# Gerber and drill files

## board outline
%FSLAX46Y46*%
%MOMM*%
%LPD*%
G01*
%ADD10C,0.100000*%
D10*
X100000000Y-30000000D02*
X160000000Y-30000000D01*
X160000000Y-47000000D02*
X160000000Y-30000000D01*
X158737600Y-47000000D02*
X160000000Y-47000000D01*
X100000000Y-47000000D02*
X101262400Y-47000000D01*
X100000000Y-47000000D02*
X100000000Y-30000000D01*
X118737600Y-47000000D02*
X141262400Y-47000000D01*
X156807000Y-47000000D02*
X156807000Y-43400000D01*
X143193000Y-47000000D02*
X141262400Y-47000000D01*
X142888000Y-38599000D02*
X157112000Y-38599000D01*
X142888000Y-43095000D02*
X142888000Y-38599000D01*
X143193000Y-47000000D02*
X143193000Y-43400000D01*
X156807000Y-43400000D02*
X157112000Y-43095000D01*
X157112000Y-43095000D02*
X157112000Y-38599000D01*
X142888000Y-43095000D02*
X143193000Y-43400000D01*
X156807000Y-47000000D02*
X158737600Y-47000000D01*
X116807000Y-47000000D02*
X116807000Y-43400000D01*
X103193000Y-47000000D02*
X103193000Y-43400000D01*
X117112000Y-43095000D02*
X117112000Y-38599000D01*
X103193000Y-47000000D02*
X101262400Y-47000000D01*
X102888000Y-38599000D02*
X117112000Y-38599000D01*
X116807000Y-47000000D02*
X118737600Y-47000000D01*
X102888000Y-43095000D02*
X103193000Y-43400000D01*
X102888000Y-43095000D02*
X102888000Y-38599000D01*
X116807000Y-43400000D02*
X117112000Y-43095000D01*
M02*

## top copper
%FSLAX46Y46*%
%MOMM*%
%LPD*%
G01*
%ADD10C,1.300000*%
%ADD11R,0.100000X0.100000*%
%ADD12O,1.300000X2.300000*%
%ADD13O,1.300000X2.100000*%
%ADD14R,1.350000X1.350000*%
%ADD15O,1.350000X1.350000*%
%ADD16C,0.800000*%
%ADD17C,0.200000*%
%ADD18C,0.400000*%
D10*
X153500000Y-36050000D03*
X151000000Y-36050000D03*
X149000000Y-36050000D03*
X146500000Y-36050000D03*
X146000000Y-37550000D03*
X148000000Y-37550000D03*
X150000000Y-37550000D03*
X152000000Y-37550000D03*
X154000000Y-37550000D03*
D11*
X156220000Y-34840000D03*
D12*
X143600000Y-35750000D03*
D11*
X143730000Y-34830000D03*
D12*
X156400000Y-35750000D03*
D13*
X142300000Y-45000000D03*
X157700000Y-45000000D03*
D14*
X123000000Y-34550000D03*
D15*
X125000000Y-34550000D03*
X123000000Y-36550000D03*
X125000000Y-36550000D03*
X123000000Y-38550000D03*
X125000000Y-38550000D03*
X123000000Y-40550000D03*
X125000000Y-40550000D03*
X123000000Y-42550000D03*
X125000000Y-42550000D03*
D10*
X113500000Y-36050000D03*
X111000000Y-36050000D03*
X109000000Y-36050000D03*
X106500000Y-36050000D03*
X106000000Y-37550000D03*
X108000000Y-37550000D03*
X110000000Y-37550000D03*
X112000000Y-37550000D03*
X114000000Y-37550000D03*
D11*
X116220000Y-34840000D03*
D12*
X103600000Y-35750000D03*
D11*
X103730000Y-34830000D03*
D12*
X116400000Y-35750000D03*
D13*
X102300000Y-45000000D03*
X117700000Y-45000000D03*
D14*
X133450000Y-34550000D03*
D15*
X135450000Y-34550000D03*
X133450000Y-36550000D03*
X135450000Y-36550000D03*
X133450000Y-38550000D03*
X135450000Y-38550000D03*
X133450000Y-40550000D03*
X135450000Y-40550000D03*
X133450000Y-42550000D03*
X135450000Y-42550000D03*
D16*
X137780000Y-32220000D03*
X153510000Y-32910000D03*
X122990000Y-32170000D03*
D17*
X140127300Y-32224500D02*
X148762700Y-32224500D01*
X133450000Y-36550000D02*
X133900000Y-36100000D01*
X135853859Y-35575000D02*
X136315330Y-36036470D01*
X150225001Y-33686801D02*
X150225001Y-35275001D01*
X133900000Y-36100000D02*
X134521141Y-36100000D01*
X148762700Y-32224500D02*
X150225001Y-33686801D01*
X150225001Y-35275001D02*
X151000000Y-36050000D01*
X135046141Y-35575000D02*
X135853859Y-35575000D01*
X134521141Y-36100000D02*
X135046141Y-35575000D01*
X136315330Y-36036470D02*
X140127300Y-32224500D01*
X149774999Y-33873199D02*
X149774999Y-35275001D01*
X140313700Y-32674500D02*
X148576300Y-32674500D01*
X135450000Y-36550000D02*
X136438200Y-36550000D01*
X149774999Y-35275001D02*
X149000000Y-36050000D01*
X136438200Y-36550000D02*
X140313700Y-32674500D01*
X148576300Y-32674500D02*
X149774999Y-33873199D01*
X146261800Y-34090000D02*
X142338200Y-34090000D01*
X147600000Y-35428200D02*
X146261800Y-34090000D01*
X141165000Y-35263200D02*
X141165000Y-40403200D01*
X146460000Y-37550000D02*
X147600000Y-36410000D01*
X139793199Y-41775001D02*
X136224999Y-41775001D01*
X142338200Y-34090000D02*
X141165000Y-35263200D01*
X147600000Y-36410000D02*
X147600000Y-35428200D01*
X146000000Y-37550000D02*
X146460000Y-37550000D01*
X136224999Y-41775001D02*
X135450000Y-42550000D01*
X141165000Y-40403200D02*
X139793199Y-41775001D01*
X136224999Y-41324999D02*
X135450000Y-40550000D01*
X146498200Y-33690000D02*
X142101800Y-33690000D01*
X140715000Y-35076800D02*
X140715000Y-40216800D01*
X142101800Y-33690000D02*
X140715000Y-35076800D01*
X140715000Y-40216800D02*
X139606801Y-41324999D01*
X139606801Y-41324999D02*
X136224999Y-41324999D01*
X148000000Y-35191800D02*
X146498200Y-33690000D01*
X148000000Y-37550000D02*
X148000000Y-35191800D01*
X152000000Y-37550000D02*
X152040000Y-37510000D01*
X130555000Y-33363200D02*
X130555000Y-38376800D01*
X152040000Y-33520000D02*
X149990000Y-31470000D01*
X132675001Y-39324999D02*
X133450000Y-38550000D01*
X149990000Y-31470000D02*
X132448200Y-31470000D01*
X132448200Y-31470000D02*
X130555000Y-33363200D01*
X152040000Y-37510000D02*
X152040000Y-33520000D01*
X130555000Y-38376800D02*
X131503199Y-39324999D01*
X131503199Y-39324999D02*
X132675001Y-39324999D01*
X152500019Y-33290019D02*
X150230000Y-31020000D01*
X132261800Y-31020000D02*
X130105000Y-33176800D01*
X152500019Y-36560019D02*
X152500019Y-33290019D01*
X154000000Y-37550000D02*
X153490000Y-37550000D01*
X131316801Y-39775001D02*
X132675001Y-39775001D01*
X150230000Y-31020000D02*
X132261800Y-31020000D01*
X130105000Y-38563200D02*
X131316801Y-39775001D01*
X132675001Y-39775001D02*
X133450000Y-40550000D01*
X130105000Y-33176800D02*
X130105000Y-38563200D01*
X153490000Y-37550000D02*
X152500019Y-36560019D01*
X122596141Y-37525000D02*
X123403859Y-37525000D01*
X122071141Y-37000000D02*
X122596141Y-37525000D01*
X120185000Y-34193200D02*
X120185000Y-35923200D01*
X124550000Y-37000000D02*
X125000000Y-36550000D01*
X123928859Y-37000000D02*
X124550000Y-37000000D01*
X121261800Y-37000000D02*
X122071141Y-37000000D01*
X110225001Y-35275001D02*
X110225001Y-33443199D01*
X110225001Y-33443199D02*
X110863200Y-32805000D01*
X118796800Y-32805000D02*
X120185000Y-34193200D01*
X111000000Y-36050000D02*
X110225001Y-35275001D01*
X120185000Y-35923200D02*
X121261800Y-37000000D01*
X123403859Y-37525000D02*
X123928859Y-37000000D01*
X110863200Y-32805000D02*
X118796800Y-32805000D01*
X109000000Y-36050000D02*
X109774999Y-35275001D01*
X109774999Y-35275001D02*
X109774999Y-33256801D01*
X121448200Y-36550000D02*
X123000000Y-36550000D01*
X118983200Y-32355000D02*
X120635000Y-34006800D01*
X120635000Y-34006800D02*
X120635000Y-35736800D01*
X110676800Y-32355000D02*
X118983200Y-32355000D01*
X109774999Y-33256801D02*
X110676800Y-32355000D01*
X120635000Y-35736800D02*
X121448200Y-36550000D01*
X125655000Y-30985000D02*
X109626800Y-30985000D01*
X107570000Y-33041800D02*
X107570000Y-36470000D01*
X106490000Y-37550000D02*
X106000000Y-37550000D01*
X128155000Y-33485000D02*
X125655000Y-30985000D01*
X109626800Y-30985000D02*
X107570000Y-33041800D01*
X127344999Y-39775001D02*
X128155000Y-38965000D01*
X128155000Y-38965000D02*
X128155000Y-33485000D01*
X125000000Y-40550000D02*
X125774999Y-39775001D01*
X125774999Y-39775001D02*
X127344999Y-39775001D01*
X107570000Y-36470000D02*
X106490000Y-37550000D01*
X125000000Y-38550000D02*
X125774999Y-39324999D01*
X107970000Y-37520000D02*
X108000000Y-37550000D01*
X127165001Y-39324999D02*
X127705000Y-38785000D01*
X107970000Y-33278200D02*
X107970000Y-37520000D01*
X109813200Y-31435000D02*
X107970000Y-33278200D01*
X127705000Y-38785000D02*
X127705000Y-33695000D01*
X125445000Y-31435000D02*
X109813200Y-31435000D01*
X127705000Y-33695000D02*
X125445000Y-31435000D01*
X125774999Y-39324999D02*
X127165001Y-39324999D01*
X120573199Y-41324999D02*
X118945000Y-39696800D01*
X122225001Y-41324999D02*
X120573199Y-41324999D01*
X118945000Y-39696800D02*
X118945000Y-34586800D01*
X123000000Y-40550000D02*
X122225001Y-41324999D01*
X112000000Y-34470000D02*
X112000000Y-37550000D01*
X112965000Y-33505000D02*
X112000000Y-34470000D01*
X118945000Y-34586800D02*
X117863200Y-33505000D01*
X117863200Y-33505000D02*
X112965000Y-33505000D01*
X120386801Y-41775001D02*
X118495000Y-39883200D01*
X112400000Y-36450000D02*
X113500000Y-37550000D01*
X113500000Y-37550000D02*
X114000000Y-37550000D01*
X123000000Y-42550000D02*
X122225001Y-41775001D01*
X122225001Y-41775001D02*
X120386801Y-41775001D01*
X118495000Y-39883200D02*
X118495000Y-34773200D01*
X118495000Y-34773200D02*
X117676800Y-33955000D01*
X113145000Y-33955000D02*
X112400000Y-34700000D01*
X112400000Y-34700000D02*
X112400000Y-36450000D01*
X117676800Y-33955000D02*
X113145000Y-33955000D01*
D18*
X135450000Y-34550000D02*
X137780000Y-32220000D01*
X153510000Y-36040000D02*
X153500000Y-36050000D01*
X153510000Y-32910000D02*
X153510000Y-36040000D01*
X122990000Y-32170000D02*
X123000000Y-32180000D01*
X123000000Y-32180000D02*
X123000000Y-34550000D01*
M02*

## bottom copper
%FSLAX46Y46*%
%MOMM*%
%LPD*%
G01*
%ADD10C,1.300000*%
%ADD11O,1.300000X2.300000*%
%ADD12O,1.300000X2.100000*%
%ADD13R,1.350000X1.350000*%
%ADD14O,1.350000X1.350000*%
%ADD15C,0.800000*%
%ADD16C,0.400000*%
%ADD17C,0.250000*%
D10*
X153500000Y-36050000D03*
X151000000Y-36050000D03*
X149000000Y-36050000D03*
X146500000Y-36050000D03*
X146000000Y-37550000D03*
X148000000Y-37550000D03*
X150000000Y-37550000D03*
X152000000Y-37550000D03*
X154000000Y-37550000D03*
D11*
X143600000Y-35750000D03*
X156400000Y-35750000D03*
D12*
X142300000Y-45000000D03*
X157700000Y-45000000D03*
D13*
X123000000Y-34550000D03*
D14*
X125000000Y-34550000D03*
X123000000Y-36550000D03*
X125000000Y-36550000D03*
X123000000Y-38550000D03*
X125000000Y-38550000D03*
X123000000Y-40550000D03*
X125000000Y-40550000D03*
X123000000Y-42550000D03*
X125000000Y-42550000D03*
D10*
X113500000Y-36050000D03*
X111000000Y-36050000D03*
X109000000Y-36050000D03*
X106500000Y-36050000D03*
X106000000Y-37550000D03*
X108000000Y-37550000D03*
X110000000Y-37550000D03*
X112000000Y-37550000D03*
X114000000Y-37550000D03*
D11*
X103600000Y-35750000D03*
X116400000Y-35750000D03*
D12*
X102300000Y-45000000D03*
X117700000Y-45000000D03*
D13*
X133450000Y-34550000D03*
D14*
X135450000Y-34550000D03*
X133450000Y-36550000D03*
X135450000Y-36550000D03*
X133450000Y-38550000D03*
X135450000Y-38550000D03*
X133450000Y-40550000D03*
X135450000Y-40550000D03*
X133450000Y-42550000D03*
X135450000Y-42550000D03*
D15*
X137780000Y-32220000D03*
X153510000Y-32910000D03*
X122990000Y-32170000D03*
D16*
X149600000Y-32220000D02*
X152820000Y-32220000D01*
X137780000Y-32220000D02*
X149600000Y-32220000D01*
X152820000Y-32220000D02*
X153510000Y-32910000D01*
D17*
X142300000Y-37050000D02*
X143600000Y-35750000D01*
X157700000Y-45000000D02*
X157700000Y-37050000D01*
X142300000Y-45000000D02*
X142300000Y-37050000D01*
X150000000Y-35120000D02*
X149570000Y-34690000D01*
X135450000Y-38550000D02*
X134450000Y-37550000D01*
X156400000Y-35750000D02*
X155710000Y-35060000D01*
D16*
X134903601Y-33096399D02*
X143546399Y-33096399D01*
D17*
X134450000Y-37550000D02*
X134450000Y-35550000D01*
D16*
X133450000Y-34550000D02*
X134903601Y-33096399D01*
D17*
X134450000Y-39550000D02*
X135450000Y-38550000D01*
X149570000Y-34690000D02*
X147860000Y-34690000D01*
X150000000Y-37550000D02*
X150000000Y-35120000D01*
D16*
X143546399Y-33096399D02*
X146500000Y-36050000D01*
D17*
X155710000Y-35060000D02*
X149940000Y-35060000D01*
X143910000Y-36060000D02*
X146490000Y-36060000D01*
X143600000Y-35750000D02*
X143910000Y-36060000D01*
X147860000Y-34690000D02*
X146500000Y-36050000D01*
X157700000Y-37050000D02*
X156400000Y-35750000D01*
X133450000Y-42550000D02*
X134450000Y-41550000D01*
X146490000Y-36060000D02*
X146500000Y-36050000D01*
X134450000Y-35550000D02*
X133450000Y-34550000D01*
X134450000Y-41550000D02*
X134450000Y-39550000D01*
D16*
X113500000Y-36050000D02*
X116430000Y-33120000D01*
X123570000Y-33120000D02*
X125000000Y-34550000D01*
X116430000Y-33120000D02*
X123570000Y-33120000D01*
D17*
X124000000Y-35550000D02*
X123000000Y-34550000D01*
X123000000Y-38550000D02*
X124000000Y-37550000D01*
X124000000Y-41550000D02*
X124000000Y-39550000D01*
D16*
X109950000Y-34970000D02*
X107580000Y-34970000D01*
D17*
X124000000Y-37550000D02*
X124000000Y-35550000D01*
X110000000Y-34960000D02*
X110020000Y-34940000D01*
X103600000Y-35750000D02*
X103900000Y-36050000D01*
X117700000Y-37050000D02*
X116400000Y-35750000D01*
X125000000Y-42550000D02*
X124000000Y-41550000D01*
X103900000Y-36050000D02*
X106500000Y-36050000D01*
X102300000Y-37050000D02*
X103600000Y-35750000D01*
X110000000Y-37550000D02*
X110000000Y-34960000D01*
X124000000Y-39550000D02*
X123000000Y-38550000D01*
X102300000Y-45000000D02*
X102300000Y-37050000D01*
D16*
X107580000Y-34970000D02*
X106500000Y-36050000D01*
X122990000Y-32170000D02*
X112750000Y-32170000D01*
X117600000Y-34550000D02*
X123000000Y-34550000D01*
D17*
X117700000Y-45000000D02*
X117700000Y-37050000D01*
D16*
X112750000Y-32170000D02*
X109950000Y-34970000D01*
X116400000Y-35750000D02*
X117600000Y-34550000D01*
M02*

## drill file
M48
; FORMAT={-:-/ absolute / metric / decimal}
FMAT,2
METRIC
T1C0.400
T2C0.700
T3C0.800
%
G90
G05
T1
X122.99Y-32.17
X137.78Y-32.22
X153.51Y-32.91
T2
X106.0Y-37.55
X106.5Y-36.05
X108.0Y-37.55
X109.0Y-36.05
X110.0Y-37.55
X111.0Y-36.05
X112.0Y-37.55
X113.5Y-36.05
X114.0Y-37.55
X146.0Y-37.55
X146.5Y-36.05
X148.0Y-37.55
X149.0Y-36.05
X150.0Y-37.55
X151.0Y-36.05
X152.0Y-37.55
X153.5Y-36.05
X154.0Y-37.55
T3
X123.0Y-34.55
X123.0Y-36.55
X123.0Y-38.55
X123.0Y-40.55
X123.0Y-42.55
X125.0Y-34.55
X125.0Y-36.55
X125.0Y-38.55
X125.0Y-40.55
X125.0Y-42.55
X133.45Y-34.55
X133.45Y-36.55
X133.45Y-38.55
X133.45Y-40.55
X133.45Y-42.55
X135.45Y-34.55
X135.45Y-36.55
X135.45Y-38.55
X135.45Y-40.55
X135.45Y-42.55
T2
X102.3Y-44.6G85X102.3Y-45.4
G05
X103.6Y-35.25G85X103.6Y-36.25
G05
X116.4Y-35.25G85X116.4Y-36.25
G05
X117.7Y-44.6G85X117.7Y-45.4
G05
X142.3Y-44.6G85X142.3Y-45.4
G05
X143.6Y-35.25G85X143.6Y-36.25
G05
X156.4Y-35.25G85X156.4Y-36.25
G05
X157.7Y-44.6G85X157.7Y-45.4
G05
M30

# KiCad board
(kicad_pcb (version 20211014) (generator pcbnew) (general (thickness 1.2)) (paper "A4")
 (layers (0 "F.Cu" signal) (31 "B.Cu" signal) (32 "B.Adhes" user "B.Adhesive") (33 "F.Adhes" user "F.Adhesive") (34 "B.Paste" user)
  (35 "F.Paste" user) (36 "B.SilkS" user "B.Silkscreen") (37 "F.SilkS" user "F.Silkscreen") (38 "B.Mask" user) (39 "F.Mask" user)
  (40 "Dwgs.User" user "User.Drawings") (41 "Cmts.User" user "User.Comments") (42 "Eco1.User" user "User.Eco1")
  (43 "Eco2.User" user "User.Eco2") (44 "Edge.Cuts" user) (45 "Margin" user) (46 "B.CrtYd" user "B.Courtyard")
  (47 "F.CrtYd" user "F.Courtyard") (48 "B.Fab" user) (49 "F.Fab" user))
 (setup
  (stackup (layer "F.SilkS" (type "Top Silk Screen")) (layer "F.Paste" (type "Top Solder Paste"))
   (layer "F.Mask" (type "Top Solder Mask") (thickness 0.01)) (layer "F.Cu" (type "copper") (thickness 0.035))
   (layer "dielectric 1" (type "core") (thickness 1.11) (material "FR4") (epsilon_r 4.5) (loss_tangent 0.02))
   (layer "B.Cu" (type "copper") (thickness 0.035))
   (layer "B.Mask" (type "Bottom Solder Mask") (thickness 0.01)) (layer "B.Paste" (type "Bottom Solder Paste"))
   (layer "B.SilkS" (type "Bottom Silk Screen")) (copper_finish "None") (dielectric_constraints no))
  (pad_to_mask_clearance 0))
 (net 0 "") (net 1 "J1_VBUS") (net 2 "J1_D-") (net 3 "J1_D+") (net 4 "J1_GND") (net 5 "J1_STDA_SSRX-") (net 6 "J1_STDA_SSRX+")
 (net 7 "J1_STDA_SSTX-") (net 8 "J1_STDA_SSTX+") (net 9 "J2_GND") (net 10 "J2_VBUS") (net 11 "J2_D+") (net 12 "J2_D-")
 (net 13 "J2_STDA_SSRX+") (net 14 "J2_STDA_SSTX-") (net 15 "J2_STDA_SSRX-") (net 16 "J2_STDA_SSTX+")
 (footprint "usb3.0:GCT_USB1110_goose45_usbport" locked (layer "F.Cu") (at 150 45)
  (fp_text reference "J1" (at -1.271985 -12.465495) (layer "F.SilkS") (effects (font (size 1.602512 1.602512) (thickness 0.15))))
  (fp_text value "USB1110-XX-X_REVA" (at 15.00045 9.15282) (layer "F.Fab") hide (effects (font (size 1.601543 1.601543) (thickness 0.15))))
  (fp_line (start 6.807 2) (end 6.807 -1.6) (layer "Edge.Cuts") (width 0.1))
  (fp_line (start -6.807 2) (end -8.7376 2) (layer "Edge.Cuts") (width 0.1))
  (fp_line (start -7.112 -6.401) (end 7.112 -6.401) (layer "Edge.Cuts") (width 0.1))
  (fp_line (start -7.112 -1.905) (end -7.112 -6.401) (layer "Edge.Cuts") (width 0.1))
  (fp_line (start -6.807 2) (end -6.807 -1.6) (layer "Edge.Cuts") (width 0.1))
  (fp_line (start 6.807 -1.6) (end 7.112 -1.905) (layer "Edge.Cuts") (width 0.1))
  (fp_line (start 7.112 -1.905) (end 7.112 -6.401) (layer "Edge.Cuts") (width 0.1))
  (fp_line (start -7.112 -1.905) (end -6.807 -1.6) (layer "Edge.Cuts") (width 0.1))
  (fp_line (start 6.807 2) (end 8.7376 2) (layer "Edge.Cuts") (width 0.1))
  (pad "1" thru_hole circle locked (at 3.5 -8.95) (size 1.3 1.3) (drill 0.7) (layers *.Cu *.Mask) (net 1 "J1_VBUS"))
  (pad "2" thru_hole circle locked (at 1 -8.95) (size 1.3 1.3) (drill 0.7) (layers *.Cu *.Mask) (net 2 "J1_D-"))
  (pad "3" thru_hole circle locked (at -1 -8.95) (size 1.3 1.3) (drill 0.7) (layers *.Cu *.Mask) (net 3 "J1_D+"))
  (pad "4" thru_hole circle locked (at -3.5 -8.95) (size 1.3 1.3) (drill 0.7) (layers *.Cu *.Mask) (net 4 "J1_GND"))
  (pad "5" thru_hole circle locked (at -4 -7.45) (size 1.3 1.3) (drill 0.7) (layers *.Cu *.Mask) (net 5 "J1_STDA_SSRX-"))
  (pad "6" thru_hole circle locked (at -2 -7.45) (size 1.3 1.3) (drill 0.7) (layers *.Cu *.Mask) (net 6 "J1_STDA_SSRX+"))
  (pad "7" thru_hole circle locked (at 0 -7.45) (size 1.3 1.3) (drill 0.7) (layers *.Cu *.Mask) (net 4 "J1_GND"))
  (pad "8" thru_hole circle locked (at 2 -7.45) (size 1.3 1.3) (drill 0.7) (layers *.Cu *.Mask) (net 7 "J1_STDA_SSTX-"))
  (pad "9" thru_hole circle locked (at 4 -7.45) (size 1.3 1.3) (drill 0.7) (layers *.Cu *.Mask) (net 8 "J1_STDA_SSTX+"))
  (pad "10" smd rect locked (at 6.22 -10.16) (size 0.1 0.1) (layers "F.Cu") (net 4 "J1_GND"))
  (pad "10" thru_hole oval locked (at -6.4 -9.25) (size 1.3 2.3) (drill oval 0.7 1.7) (layers *.Cu *.Mask) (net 4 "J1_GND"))
  (pad "11" smd rect locked (at -6.27 -10.17) (size 0.1 0.1) (layers "F.Cu") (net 4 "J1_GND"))
  (pad "11" thru_hole oval locked (at 6.4 -9.25) (size 1.3 2.3) (drill oval 0.7 1.7) (layers *.Cu *.Mask) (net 4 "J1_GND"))
  (pad "12" thru_hole oval locked (at -7.7 0) (size 1.3 2.1) (drill oval 0.7 1.5) (layers *.Cu *.Mask) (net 4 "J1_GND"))
  (pad "13" thru_hole oval locked (at 7.7 0) (size 1.3 2.1) (drill oval 0.7 1.5) (layers *.Cu *.Mask) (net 4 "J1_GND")))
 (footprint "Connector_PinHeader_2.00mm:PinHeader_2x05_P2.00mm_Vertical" (layer "F.Cu") (at 123 34.55)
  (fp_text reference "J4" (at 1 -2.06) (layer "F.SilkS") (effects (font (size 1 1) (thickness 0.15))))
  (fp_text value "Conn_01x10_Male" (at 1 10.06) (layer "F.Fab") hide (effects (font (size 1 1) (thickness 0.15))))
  (pad "1" thru_hole rect (at 0 0) (size 1.35 1.35) (drill 0.8) (layers *.Cu *.Mask) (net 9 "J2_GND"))
  (pad "2" thru_hole oval (at 2 0) (size 1.35 1.35) (drill 0.8) (layers *.Cu *.Mask) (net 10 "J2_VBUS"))
  (pad "3" thru_hole oval (at 0 2) (size 1.35 1.35) (drill 0.8) (layers *.Cu *.Mask) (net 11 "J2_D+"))
  (pad "4" thru_hole oval (at 2 2) (size 1.35 1.35) (drill 0.8) (layers *.Cu *.Mask) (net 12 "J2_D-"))
  (pad "5" thru_hole oval (at 0 4) (size 1.35 1.35) (drill 0.8) (layers *.Cu *.Mask) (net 9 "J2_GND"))
  (pad "6" thru_hole oval (at 2 4) (size 1.35 1.35) (drill 0.8) (layers *.Cu *.Mask) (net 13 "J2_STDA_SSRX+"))
  (pad "7" thru_hole oval (at 0 6) (size 1.35 1.35) (drill 0.8) (layers *.Cu *.Mask) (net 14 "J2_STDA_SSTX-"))
  (pad "8" thru_hole oval (at 2 6) (size 1.35 1.35) (drill 0.8) (layers *.Cu *.Mask) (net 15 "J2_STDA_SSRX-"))
  (pad "9" thru_hole oval (at 0 8) (size 1.35 1.35) (drill 0.8) (layers *.Cu *.Mask) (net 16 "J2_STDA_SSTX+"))
  (pad "10" thru_hole oval (at 2 8) (size 1.35 1.35) (drill 0.8) (layers *.Cu *.Mask) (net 9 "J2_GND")))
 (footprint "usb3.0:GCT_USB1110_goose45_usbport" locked (layer "F.Cu") (at 110 45)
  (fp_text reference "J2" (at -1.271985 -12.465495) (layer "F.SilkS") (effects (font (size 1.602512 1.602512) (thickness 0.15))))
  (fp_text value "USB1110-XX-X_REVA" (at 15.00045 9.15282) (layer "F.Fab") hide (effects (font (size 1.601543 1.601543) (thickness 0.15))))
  (fp_line (start 6.807 2) (end 6.807 -1.6) (layer "Edge.Cuts") (width 0.1))
  (fp_line (start -6.807 2) (end -6.807 -1.6) (layer "Edge.Cuts") (width 0.1))
  (fp_line (start 7.112 -1.905) (end 7.112 -6.401) (layer "Edge.Cuts") (width 0.1))
  (fp_line (start -6.807 2) (end -8.7376 2) (layer "Edge.Cuts") (width 0.1))
  (fp_line (start -7.112 -6.401) (end 7.112 -6.401) (layer "Edge.Cuts") (width 0.1))
  (fp_line (start 6.807 2) (end 8.7376 2) (layer "Edge.Cuts") (width 0.1))
  (fp_line (start -7.112 -1.905) (end -6.807 -1.6) (layer "Edge.Cuts") (width 0.1))
  (fp_line (start -7.112 -1.905) (end -7.112 -6.401) (layer "Edge.Cuts") (width 0.1))
  (fp_line (start 6.807 -1.6) (end 7.112 -1.905) (layer "Edge.Cuts") (width 0.1))
  (pad "1" thru_hole circle locked (at 3.5 -8.95) (size 1.3 1.3) (drill 0.7) (layers *.Cu *.Mask) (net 10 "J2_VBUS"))
  (pad "2" thru_hole circle locked (at 1 -8.95) (size 1.3 1.3) (drill 0.7) (layers *.Cu *.Mask) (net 12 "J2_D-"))
  (pad "3" thru_hole circle locked (at -1 -8.95) (size 1.3 1.3) (drill 0.7) (layers *.Cu *.Mask) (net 11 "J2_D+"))
  (pad "4" thru_hole circle locked (at -3.5 -8.95) (size 1.3 1.3) (drill 0.7) (layers *.Cu *.Mask) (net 9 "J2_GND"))
  (pad "5" thru_hole circle locked (at -4 -7.45) (size 1.3 1.3) (drill 0.7) (layers *.Cu *.Mask) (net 15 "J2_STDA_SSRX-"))
  (pad "6" thru_hole circle locked (at -2 -7.45) (size 1.3 1.3) (drill 0.7) (layers *.Cu *.Mask) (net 13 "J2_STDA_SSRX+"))
  (pad "7" thru_hole circle locked (at 0 -7.45) (size 1.3 1.3) (drill 0.7) (layers *.Cu *.Mask) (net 9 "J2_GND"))
  (pad "8" thru_hole circle locked (at 2 -7.45) (size 1.3 1.3) (drill 0.7) (layers *.Cu *.Mask) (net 14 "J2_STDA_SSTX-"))
  (pad "9" thru_hole circle locked (at 4 -7.45) (size 1.3 1.3) (drill 0.7) (layers *.Cu *.Mask) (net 16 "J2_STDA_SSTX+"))
  (pad "10" smd rect locked (at 6.22 -10.16) (size 0.1 0.1) (layers "F.Cu") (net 9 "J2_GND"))
  (pad "10" thru_hole oval locked (at -6.4 -9.25) (size 1.3 2.3) (drill oval 0.7 1.7) (layers *.Cu *.Mask) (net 9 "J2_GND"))
  (pad "11" smd rect locked (at -6.27 -10.17) (size 0.1 0.1) (layers "F.Cu") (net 9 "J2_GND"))
  (pad "11" thru_hole oval locked (at 6.4 -9.25) (size 1.3 2.3) (drill oval 0.7 1.7) (layers *.Cu *.Mask) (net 9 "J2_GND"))
  (pad "12" thru_hole oval locked (at -7.7 0) (size 1.3 2.1) (drill oval 0.7 1.5) (layers *.Cu *.Mask) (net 9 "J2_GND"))
  (pad "13" thru_hole oval locked (at 7.7 0) (size 1.3 2.1) (drill oval 0.7 1.5) (layers *.Cu *.Mask) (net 9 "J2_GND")))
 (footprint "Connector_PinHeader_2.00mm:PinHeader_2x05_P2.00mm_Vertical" (layer "F.Cu") (at 133.45 34.55)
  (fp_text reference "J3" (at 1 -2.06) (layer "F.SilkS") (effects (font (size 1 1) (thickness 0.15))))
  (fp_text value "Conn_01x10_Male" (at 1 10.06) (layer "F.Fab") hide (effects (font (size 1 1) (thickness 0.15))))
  (pad "1" thru_hole rect (at 0 0) (size 1.35 1.35) (drill 0.8) (layers *.Cu *.Mask) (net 4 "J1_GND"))
  (pad "2" thru_hole oval (at 2 0) (size 1.35 1.35) (drill 0.8) (layers *.Cu *.Mask) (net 1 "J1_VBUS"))
  (pad "3" thru_hole oval (at 0 2) (size 1.35 1.35) (drill 0.8) (layers *.Cu *.Mask) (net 2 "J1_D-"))
  (pad "4" thru_hole oval (at 2 2) (size 1.35 1.35) (drill 0.8) (layers *.Cu *.Mask) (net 3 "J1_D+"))
  (pad "5" thru_hole oval (at 0 4) (size 1.35 1.35) (drill 0.8) (layers *.Cu *.Mask) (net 7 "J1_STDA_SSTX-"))
  (pad "6" thru_hole oval (at 2 4) (size 1.35 1.35) (drill 0.8) (layers *.Cu *.Mask) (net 4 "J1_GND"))
  (pad "7" thru_hole oval (at 0 6) (size 1.35 1.35) (drill 0.8) (layers *.Cu *.Mask) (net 8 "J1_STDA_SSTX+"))
  (pad "8" thru_hole oval (at 2 6) (size 1.35 1.35) (drill 0.8) (layers *.Cu *.Mask) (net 6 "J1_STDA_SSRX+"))
  (pad "9" thru_hole oval (at 0 8) (size 1.35 1.35) (drill 0.8) (layers *.Cu *.Mask) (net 4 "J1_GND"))
  (pad "10" thru_hole oval (at 2 8) (size 1.35 1.35) (drill 0.8) (layers *.Cu *.Mask) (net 5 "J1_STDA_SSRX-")))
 (gr_line (start 100 30) (end 160 30) (layer "Edge.Cuts") (width 0.1))
 (gr_line (start 160 47) (end 160 30) (layer "Edge.Cuts") (width 0.1))
 (gr_line locked (start 158.7376 47) (end 160 47) (layer "Edge.Cuts") (width 0.1))
 (gr_line locked (start 100 47) (end 101.2624 47) (layer "Edge.Cuts") (width 0.1))
 (gr_line (start 100 47) (end 100 30) (layer "Edge.Cuts") (width 0.1))
 (gr_line locked (start 118.7376 47) (end 141.2624 47) (layer "Edge.Cuts") (width 0.1))
 (segment (start 140.1273 32.2245) (end 148.7627 32.2245) (width 0.2) (layer "F.Cu") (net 2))
 (segment (start 133.45 36.55) (end 133.9 36.1) (width 0.2) (layer "F.Cu") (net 2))
 (segment (start 135.853859 35.575) (end 136.31533 36.03647) (width 0.2) (layer "F.Cu") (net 2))
 (segment (start 150.225001 33.686801) (end 150.225001 35.275001) (width 0.2) (layer "F.Cu") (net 2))
 (segment (start 133.9 36.1) (end 134.521141 36.1) (width 0.2) (layer "F.Cu") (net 2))
 (segment (start 148.7627 32.2245) (end 150.225001 33.686801) (width 0.2) (layer "F.Cu") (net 2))
 (segment (start 150.225001 35.275001) (end 151 36.05) (width 0.2) (layer "F.Cu") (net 2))
 (segment (start 135.046141 35.575) (end 135.853859 35.575) (width 0.2) (layer "F.Cu") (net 2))
 (segment (start 134.521141 36.1) (end 135.046141 35.575) (width 0.2) (layer "F.Cu") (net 2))
 (segment (start 136.31533 36.03647) (end 140.1273 32.2245) (width 0.2) (layer "F.Cu") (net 2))
 (segment (start 149.774999 33.873199) (end 149.774999 35.275001) (width 0.2) (layer "F.Cu") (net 3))
 (segment (start 140.3137 32.6745) (end 148.5763 32.6745) (width 0.2) (layer "F.Cu") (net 3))
 (segment (start 135.45 36.55) (end 136.4382 36.55) (width 0.2) (layer "F.Cu") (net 3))
 (segment (start 149.774999 35.275001) (end 149 36.05) (width 0.2) (layer "F.Cu") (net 3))
 (segment (start 136.4382 36.55) (end 140.3137 32.6745) (width 0.2) (layer "F.Cu") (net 3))
 (segment (start 148.5763 32.6745) (end 149.774999 33.873199) (width 0.2) (layer "F.Cu") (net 3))
 (segment (start 146.2618 34.09) (end 142.3382 34.09) (width 0.2) (layer "F.Cu") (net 5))
 (segment (start 147.6 35.4282) (end 146.2618 34.09) (width 0.2) (layer "F.Cu") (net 5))
 (segment (start 141.165 35.2632) (end 141.165 40.4032) (width 0.2) (layer "F.Cu") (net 5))
 (segment (start 146.46 37.55) (end 147.6 36.41) (width 0.2) (layer "F.Cu") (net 5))
 (segment (start 139.793199 41.775001) (end 136.224999 41.775001) (width 0.2) (layer "F.Cu") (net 5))
 (segment (start 142.3382 34.09) (end 141.165 35.2632) (width 0.2) (layer "F.Cu") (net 5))
 (segment (start 147.6 36.41) (end 147.6 35.4282) (width 0.2) (layer "F.Cu") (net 5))
 (segment (start 146 37.55) (end 146.46 37.55) (width 0.2) (layer "F.Cu") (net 5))
 (segment (start 136.224999 41.775001) (end 135.45 42.55) (width 0.2) (layer "F.Cu") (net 5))
 (segment (start 141.165 40.4032) (end 139.793199 41.775001) (width 0.2) (layer "F.Cu") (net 5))
 (segment (start 136.224999 41.324999) (end 135.45 40.55) (width 0.2) (layer "F.Cu") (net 6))
 (segment (start 146.4982 33.69) (end 142.1018 33.69) (width 0.2) (layer "F.Cu") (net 6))
 (segment (start 140.715 35.0768) (end 140.715 40.2168) (width 0.2) (layer "F.Cu") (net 6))
 (segment (start 142.1018 33.69) (end 140.715 35.0768) (width 0.2) (layer "F.Cu") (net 6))
 (segment (start 140.715 40.2168) (end 139.606801 41.324999) (width 0.2) (layer "F.Cu") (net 6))
 (segment (start 139.606801 41.324999) (end 136.224999 41.324999) (width 0.2) (layer "F.Cu") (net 6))
 (segment (start 148 35.1918) (end 146.4982 33.69) (width 0.2) (layer "F.Cu") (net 6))
 (segment (start 148 37.55) (end 148 35.1918) (width 0.2) (layer "F.Cu") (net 6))
 (segment (start 152 37.55) (end 152.04 37.51) (width 0.2) (layer "F.Cu") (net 7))
 (segment (start 130.555 33.3632) (end 130.555 38.3768) (width 0.2) (layer "F.Cu") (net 7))
 (segment (start 152.04 33.52) (end 149.99 31.47) (width 0.2) (layer "F.Cu") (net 7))
 (segment (start 132.675001 39.324999) (end 133.45 38.55) (width 0.2) (layer "F.Cu") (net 7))
 (segment (start 149.99 31.47) (end 132.4482 31.47) (width 0.2) (layer "F.Cu") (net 7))
 (segment (start 132.4482 31.47) (end 130.555 33.3632) (width 0.2) (layer "F.Cu") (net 7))
 (segment (start 152.04 37.51) (end 152.04 33.52) (width 0.2) (layer "F.Cu") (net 7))
 (segment (start 130.555 38.3768) (end 131.503199 39.324999) (width 0.2) (layer "F.Cu") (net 7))
 (segment (start 131.503199 39.324999) (end 132.675001 39.324999) (width 0.2) (layer "F.Cu") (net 7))
 (segment (start 152.500019 33.290019) (end 150.23 31.02) (width 0.2) (layer "F.Cu") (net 8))
 (segment (start 132.2618 31.02) (end 130.105 33.1768) (width 0.2) (layer "F.Cu") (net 8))
 (segment (start 152.500019 36.560019) (end 152.500019 33.290019) (width 0.2) (layer "F.Cu") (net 8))
 (segment (start 154 37.55) (end 153.49 37.55) (width 0.2) (layer "F.Cu") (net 8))
 (segment (start 131.316801 39.775001) (end 132.675001 39.775001) (width 0.2) (layer "F.Cu") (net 8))
 (segment (start 150.23 31.02) (end 132.2618 31.02) (width 0.2) (layer "F.Cu") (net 8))
 (segment (start 130.105 38.5632) (end 131.316801 39.775001) (width 0.2) (layer "F.Cu") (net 8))
 (segment (start 132.675001 39.775001) (end 133.45 40.55) (width 0.2) (layer "F.Cu") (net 8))
 (segment (start 130.105 33.1768) (end 130.105 38.5632) (width 0.2) (layer "F.Cu") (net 8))
 (segment (start 153.49 37.55) (end 152.500019 36.560019) (width 0.2) (layer "F.Cu") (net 8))
 (segment (start 122.596141 37.525) (end 123.403859 37.525) (width 0.2) (layer "F.Cu") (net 12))
 (segment (start 122.071141 37) (end 122.596141 37.525) (width 0.2) (layer "F.Cu") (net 12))
 (segment (start 120.185 34.1932) (end 120.185 35.9232) (width 0.2) (layer "F.Cu") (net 12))
 (segment (start 124.55 37) (end 125 36.55) (width 0.2) (layer "F.Cu") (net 12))
 (segment (start 123.928859 37) (end 124.55 37) (width 0.2) (layer "F.Cu") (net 12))
 (segment (start 121.2618 37) (end 122.071141 37) (width 0.2) (layer "F.Cu") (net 12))
 (segment (start 110.225001 35.275001) (end 110.225001 33.443199) (width 0.2) (layer "F.Cu") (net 12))
 (segment (start 110.225001 33.443199) (end 110.8632 32.805) (width 0.2) (layer "F.Cu") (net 12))
 (segment (start 118.7968 32.805) (end 120.185 34.1932) (width 0.2) (layer "F.Cu") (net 12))
 (segment (start 111 36.05) (end 110.225001 35.275001) (width 0.2) (layer "F.Cu") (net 12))
 (segment (start 120.185 35.9232) (end 121.2618 37) (width 0.2) (layer "F.Cu") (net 12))
 (segment (start 123.403859 37.525) (end 123.928859 37) (width 0.2) (layer "F.Cu") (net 12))
 (segment (start 110.8632 32.805) (end 118.7968 32.805) (width 0.2) (layer "F.Cu") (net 12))
 (segment (start 109 36.05) (end 109.774999 35.275001) (width 0.2) (layer "F.Cu") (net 11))
 (segment (start 109.774999 35.275001) (end 109.774999 33.256801) (width 0.2) (layer "F.Cu") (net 11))
 (segment (start 121.4482 36.55) (end 123 36.55) (width 0.2) (layer "F.Cu") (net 11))
 (segment (start 118.9832 32.355) (end 120.635 34.0068) (width 0.2) (layer "F.Cu") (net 11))
 (segment (start 120.635 34.0068) (end 120.635 35.7368) (width 0.2) (layer "F.Cu") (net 11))
 (segment (start 110.6768 32.355) (end 118.9832 32.355) (width 0.2) (layer "F.Cu") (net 11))
 (segment (start 109.774999 33.256801) (end 110.6768 32.355) (width 0.2) (layer "F.Cu") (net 11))
 (segment (start 120.635 35.7368) (end 121.4482 36.55) (width 0.2) (layer "F.Cu") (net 11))
 (segment (start 125.655 30.985) (end 109.6268 30.985) (width 0.2) (layer "F.Cu") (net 15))
 (segment (start 107.57 33.0418) (end 107.57 36.47) (width 0.2) (layer "F.Cu") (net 15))
 (segment (start 106.49 37.55) (end 106 37.55) (width 0.2) (layer "F.Cu") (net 15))
 (segment (start 128.155 33.485) (end 125.655 30.985) (width 0.2) (layer "F.Cu") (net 15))
 (segment (start 109.6268 30.985) (end 107.57 33.0418) (width 0.2) (layer "F.Cu") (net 15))
 (segment (start 127.344999 39.775001) (end 128.155 38.965) (width 0.2) (layer "F.Cu") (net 15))
 (segment (start 128.155 38.965) (end 128.155 33.485) (width 0.2) (layer "F.Cu") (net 15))
 (segment (start 125 40.55) (end 125.774999 39.775001) (width 0.2) (layer "F.Cu") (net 15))
 (segment (start 125.774999 39.775001) (end 127.344999 39.775001) (width 0.2) (layer "F.Cu") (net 15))
 (segment (start 107.57 36.47) (end 106.49 37.55) (width 0.2) (layer "F.Cu") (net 15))
 (segment (start 125 38.55) (end 125.774999 39.324999) (width 0.2) (layer "F.Cu") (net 13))
 (segment (start 107.97 37.52) (end 108 37.55) (width 0.2) (layer "F.Cu") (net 13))
 (segment (start 127.165001 39.324999) (end 127.705 38.785) (width 0.2) (layer "F.Cu") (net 13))
 (segment (start 107.97 33.2782) (end 107.97 37.52) (width 0.2) (layer "F.Cu") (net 13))
 (segment (start 109.8132 31.435) (end 107.97 33.2782) (width 0.2) (layer "F.Cu") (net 13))
 (segment (start 127.705 38.785) (end 127.705 33.695) (width 0.2) (layer "F.Cu") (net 13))
 (segment (start 125.445 31.435) (end 109.8132 31.435) (width 0.2) (layer "F.Cu") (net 13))
 (segment (start 127.705 33.695) (end 125.445 31.435) (width 0.2) (layer "F.Cu") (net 13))
 (segment (start 125.774999 39.324999) (end 127.165001 39.324999) (width 0.2) (layer "F.Cu") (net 13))
 (segment (start 120.573199 41.324999) (end 118.945 39.6968) (width 0.2) (layer "F.Cu") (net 14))
 (segment (start 122.225001 41.324999) (end 120.573199 41.324999) (width 0.2) (layer "F.Cu") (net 14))
 (segment (start 118.945 39.6968) (end 118.945 34.5868) (width 0.2) (layer "F.Cu") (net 14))
 (segment (start 123 40.55) (end 122.225001 41.324999) (width 0.2) (layer "F.Cu") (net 14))
 (segment (start 112 34.47) (end 112 37.55) (width 0.2) (layer "F.Cu") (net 14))
 (segment (start 112.965 33.505) (end 112 34.47) (width 0.2) (layer "F.Cu") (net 14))
 (segment (start 118.945 34.5868) (end 117.8632 33.505) (width 0.2) (layer "F.Cu") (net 14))
 (segment (start 117.8632 33.505) (end 112.965 33.505) (width 0.2) (layer "F.Cu") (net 14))
 (segment (start 120.386801 41.775001) (end 118.495 39.8832) (width 0.2) (layer "F.Cu") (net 16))
 (segment (start 112.4 36.45) (end 113.5 37.55) (width 0.2) (layer "F.Cu") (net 16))
 (segment (start 113.5 37.55) (end 114 37.55) (width 0.2) (layer "F.Cu") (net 16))
 (segment (start 123 42.55) (end 122.225001 41.775001) (width 0.2) (layer "F.Cu") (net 16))
 (segment (start 122.225001 41.775001) (end 120.386801 41.775001) (width 0.2) (layer "F.Cu") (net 16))
 (segment (start 118.495 39.8832) (end 118.495 34.7732) (width 0.2) (layer "F.Cu") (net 16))
 (segment (start 118.495 34.7732) (end 117.6768 33.955) (width 0.2) (layer "F.Cu") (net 16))
 (segment (start 113.145 33.955) (end 112.4 34.7) (width 0.2) (layer "F.Cu") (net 16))
 (segment (start 112.4 34.7) (end 112.4 36.45) (width 0.2) (layer "F.Cu") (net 16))
 (segment (start 117.6768 33.955) (end 113.145 33.955) (width 0.2) (layer "F.Cu") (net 16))
 (segment (start 135.45 34.55) (end 137.78 32.22) (width 0.4) (layer "F.Cu") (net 1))
 (segment (start 153.51 36.04) (end 153.5 36.05) (width 0.4) (layer "F.Cu") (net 1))
 (segment (start 153.51 32.91) (end 153.51 36.04) (width 0.4) (layer "F.Cu") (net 1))
 (via (at 137.78 32.22) (size 0.8) (drill 0.4) (layers "F.Cu" "B.Cu") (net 1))
 (via (at 153.51 32.91) (size 0.8) (drill 0.4) (layers "F.Cu" "B.Cu") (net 1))
 (segment (start 149.6 32.22) (end 152.82 32.22) (width 0.4) (layer "B.Cu") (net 1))
 (segment (start 137.78 32.22) (end 149.6 32.22) (width 0.4) (layer "B.Cu") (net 1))
 (segment (start 152.82 32.22) (end 153.51 32.91) (width 0.4) (layer "B.Cu") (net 1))
 (segment (start 142.3 37.05) (end 143.6 35.75) (width 0.25) (layer "B.Cu") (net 4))
 (segment (start 157.7 45) (end 157.7 37.05) (width 0.25) (layer "B.Cu") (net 4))
 (segment (start 142.3 45) (end 142.3 37.05) (width 0.25) (layer "B.Cu") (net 4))
 (segment (start 150 35.12) (end 149.57 34.69) (width 0.25) (layer "B.Cu") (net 4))
 (segment (start 135.45 38.55) (end 134.45 37.55) (width 0.25) (layer "B.Cu") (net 4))
 (segment (start 156.4 35.75) (end 155.71 35.06) (width 0.25) (layer "B.Cu") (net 4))
 (segment (start 134.903601 33.096399) (end 143.546399 33.096399) (width 0.4) (layer "B.Cu") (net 4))
 (segment (start 134.45 37.55) (end 134.45 35.55) (width 0.25) (layer "B.Cu") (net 4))
 (segment (start 133.45 34.55) (end 134.903601 33.096399) (width 0.4) (layer "B.Cu") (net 4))
 (segment (start 134.45 39.55) (end 135.45 38.55) (width 0.25) (layer "B.Cu") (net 4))
 (segment (start 149.57 34.69) (end 147.86 34.69) (width 0.25) (layer "B.Cu") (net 4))
 (segment (start 150 37.55) (end 150 35.12) (width 0.25) (layer "B.Cu") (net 4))
 (segment (start 143.546399 33.096399) (end 146.5 36.05) (width 0.4) (layer "B.Cu") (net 4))
 (segment (start 155.71 35.06) (end 149.94 35.06) (width 0.25) (layer "B.Cu") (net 4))
 (segment (start 143.91 36.06) (end 146.49 36.06) (width 0.25) (layer "B.Cu") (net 4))
 (segment (start 143.6 35.75) (end 143.91 36.06) (width 0.25) (layer "B.Cu") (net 4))
 (segment (start 147.86 34.69) (end 146.5 36.05) (width 0.25) (layer "B.Cu") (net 4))
 (segment (start 157.7 37.05) (end 156.4 35.75) (width 0.25) (layer "B.Cu") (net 4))
 (segment (start 133.45 42.55) (end 134.45 41.55) (width 0.25) (layer "B.Cu") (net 4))
 (segment (start 146.49 36.06) (end 146.5 36.05) (width 0.25) (layer "B.Cu") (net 4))
 (segment (start 134.45 35.55) (end 133.45 34.55) (width 0.25) (layer "B.Cu") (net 4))
 (segment (start 134.45 41.55) (end 134.45 39.55) (width 0.25) (layer "B.Cu") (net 4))
 (segment (start 113.5 36.05) (end 116.43 33.12) (width 0.4) (layer "B.Cu") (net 10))
 (segment (start 123.57 33.12) (end 125 34.55) (width 0.4) (layer "B.Cu") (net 10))
 (segment (start 116.43 33.12) (end 123.57 33.12) (width 0.4) (layer "B.Cu") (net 10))
 (segment (start 122.99 32.17) (end 123 32.18) (width 0.4) (layer "F.Cu") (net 9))
 (segment (start 123 32.18) (end 123 34.55) (width 0.4) (layer "F.Cu") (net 9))
 (via (at 122.99 32.17) (size 0.8) (drill 0.4) (layers "F.Cu" "B.Cu") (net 9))
 (segment (start 124 35.55) (end 123 34.55) (width 0.25) (layer "B.Cu") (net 9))
 (segment (start 123 38.55) (end 124 37.55) (width 0.25) (layer "B.Cu") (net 9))
 (segment (start 124 41.55) (end 124 39.55) (width 0.25) (layer "B.Cu") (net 9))
 (segment (start 109.95 34.97) (end 107.58 34.97) (width 0.4) (layer "B.Cu") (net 9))
 (segment (start 124 37.55) (end 124 35.55) (width 0.25) (layer "B.Cu") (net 9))
 (segment (start 110 34.96) (end 110.02 34.94) (width 0.25) (layer "B.Cu") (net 9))
 (segment (start 103.6 35.75) (end 103.9 36.05) (width 0.25) (layer "B.Cu") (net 9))
 (segment (start 117.7 37.05) (end 116.4 35.75) (width 0.25) (layer "B.Cu") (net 9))
 (segment (start 125 42.55) (end 124 41.55) (width 0.25) (layer "B.Cu") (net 9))
 (segment (start 103.9 36.05) (end 106.5 36.05) (width 0.25) (layer "B.Cu") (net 9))
 (segment (start 102.3 37.05) (end 103.6 35.75) (width 0.25) (layer "B.Cu") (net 9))
 (segment (start 110 37.55) (end 110 34.96) (width 0.25) (layer "B.Cu") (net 9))
 (segment (start 124 39.55) (end 123 38.55) (width 0.25) (layer "B.Cu") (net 9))
 (segment (start 102.3 45) (end 102.3 37.05) (width 0.25) (layer "B.Cu") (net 9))
 (segment (start 107.58 34.97) (end 106.5 36.05) (width 0.4) (layer "B.Cu") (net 9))
 (segment (start 122.99 32.17) (end 112.75 32.17) (width 0.4) (layer "B.Cu") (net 9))
 (segment (start 117.6 34.55) (end 123 34.55) (width 0.4) (layer "B.Cu") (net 9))
 (segment (start 117.7 45) (end 117.7 37.05) (width 0.25) (layer "B.Cu") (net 9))
 (segment (start 112.75 32.17) (end 109.95 34.97) (width 0.4) (layer "B.Cu") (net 9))
 (segment (start 116.4 35.75) (end 117.6 34.55) (width 0.4) (layer "B.Cu") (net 9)))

